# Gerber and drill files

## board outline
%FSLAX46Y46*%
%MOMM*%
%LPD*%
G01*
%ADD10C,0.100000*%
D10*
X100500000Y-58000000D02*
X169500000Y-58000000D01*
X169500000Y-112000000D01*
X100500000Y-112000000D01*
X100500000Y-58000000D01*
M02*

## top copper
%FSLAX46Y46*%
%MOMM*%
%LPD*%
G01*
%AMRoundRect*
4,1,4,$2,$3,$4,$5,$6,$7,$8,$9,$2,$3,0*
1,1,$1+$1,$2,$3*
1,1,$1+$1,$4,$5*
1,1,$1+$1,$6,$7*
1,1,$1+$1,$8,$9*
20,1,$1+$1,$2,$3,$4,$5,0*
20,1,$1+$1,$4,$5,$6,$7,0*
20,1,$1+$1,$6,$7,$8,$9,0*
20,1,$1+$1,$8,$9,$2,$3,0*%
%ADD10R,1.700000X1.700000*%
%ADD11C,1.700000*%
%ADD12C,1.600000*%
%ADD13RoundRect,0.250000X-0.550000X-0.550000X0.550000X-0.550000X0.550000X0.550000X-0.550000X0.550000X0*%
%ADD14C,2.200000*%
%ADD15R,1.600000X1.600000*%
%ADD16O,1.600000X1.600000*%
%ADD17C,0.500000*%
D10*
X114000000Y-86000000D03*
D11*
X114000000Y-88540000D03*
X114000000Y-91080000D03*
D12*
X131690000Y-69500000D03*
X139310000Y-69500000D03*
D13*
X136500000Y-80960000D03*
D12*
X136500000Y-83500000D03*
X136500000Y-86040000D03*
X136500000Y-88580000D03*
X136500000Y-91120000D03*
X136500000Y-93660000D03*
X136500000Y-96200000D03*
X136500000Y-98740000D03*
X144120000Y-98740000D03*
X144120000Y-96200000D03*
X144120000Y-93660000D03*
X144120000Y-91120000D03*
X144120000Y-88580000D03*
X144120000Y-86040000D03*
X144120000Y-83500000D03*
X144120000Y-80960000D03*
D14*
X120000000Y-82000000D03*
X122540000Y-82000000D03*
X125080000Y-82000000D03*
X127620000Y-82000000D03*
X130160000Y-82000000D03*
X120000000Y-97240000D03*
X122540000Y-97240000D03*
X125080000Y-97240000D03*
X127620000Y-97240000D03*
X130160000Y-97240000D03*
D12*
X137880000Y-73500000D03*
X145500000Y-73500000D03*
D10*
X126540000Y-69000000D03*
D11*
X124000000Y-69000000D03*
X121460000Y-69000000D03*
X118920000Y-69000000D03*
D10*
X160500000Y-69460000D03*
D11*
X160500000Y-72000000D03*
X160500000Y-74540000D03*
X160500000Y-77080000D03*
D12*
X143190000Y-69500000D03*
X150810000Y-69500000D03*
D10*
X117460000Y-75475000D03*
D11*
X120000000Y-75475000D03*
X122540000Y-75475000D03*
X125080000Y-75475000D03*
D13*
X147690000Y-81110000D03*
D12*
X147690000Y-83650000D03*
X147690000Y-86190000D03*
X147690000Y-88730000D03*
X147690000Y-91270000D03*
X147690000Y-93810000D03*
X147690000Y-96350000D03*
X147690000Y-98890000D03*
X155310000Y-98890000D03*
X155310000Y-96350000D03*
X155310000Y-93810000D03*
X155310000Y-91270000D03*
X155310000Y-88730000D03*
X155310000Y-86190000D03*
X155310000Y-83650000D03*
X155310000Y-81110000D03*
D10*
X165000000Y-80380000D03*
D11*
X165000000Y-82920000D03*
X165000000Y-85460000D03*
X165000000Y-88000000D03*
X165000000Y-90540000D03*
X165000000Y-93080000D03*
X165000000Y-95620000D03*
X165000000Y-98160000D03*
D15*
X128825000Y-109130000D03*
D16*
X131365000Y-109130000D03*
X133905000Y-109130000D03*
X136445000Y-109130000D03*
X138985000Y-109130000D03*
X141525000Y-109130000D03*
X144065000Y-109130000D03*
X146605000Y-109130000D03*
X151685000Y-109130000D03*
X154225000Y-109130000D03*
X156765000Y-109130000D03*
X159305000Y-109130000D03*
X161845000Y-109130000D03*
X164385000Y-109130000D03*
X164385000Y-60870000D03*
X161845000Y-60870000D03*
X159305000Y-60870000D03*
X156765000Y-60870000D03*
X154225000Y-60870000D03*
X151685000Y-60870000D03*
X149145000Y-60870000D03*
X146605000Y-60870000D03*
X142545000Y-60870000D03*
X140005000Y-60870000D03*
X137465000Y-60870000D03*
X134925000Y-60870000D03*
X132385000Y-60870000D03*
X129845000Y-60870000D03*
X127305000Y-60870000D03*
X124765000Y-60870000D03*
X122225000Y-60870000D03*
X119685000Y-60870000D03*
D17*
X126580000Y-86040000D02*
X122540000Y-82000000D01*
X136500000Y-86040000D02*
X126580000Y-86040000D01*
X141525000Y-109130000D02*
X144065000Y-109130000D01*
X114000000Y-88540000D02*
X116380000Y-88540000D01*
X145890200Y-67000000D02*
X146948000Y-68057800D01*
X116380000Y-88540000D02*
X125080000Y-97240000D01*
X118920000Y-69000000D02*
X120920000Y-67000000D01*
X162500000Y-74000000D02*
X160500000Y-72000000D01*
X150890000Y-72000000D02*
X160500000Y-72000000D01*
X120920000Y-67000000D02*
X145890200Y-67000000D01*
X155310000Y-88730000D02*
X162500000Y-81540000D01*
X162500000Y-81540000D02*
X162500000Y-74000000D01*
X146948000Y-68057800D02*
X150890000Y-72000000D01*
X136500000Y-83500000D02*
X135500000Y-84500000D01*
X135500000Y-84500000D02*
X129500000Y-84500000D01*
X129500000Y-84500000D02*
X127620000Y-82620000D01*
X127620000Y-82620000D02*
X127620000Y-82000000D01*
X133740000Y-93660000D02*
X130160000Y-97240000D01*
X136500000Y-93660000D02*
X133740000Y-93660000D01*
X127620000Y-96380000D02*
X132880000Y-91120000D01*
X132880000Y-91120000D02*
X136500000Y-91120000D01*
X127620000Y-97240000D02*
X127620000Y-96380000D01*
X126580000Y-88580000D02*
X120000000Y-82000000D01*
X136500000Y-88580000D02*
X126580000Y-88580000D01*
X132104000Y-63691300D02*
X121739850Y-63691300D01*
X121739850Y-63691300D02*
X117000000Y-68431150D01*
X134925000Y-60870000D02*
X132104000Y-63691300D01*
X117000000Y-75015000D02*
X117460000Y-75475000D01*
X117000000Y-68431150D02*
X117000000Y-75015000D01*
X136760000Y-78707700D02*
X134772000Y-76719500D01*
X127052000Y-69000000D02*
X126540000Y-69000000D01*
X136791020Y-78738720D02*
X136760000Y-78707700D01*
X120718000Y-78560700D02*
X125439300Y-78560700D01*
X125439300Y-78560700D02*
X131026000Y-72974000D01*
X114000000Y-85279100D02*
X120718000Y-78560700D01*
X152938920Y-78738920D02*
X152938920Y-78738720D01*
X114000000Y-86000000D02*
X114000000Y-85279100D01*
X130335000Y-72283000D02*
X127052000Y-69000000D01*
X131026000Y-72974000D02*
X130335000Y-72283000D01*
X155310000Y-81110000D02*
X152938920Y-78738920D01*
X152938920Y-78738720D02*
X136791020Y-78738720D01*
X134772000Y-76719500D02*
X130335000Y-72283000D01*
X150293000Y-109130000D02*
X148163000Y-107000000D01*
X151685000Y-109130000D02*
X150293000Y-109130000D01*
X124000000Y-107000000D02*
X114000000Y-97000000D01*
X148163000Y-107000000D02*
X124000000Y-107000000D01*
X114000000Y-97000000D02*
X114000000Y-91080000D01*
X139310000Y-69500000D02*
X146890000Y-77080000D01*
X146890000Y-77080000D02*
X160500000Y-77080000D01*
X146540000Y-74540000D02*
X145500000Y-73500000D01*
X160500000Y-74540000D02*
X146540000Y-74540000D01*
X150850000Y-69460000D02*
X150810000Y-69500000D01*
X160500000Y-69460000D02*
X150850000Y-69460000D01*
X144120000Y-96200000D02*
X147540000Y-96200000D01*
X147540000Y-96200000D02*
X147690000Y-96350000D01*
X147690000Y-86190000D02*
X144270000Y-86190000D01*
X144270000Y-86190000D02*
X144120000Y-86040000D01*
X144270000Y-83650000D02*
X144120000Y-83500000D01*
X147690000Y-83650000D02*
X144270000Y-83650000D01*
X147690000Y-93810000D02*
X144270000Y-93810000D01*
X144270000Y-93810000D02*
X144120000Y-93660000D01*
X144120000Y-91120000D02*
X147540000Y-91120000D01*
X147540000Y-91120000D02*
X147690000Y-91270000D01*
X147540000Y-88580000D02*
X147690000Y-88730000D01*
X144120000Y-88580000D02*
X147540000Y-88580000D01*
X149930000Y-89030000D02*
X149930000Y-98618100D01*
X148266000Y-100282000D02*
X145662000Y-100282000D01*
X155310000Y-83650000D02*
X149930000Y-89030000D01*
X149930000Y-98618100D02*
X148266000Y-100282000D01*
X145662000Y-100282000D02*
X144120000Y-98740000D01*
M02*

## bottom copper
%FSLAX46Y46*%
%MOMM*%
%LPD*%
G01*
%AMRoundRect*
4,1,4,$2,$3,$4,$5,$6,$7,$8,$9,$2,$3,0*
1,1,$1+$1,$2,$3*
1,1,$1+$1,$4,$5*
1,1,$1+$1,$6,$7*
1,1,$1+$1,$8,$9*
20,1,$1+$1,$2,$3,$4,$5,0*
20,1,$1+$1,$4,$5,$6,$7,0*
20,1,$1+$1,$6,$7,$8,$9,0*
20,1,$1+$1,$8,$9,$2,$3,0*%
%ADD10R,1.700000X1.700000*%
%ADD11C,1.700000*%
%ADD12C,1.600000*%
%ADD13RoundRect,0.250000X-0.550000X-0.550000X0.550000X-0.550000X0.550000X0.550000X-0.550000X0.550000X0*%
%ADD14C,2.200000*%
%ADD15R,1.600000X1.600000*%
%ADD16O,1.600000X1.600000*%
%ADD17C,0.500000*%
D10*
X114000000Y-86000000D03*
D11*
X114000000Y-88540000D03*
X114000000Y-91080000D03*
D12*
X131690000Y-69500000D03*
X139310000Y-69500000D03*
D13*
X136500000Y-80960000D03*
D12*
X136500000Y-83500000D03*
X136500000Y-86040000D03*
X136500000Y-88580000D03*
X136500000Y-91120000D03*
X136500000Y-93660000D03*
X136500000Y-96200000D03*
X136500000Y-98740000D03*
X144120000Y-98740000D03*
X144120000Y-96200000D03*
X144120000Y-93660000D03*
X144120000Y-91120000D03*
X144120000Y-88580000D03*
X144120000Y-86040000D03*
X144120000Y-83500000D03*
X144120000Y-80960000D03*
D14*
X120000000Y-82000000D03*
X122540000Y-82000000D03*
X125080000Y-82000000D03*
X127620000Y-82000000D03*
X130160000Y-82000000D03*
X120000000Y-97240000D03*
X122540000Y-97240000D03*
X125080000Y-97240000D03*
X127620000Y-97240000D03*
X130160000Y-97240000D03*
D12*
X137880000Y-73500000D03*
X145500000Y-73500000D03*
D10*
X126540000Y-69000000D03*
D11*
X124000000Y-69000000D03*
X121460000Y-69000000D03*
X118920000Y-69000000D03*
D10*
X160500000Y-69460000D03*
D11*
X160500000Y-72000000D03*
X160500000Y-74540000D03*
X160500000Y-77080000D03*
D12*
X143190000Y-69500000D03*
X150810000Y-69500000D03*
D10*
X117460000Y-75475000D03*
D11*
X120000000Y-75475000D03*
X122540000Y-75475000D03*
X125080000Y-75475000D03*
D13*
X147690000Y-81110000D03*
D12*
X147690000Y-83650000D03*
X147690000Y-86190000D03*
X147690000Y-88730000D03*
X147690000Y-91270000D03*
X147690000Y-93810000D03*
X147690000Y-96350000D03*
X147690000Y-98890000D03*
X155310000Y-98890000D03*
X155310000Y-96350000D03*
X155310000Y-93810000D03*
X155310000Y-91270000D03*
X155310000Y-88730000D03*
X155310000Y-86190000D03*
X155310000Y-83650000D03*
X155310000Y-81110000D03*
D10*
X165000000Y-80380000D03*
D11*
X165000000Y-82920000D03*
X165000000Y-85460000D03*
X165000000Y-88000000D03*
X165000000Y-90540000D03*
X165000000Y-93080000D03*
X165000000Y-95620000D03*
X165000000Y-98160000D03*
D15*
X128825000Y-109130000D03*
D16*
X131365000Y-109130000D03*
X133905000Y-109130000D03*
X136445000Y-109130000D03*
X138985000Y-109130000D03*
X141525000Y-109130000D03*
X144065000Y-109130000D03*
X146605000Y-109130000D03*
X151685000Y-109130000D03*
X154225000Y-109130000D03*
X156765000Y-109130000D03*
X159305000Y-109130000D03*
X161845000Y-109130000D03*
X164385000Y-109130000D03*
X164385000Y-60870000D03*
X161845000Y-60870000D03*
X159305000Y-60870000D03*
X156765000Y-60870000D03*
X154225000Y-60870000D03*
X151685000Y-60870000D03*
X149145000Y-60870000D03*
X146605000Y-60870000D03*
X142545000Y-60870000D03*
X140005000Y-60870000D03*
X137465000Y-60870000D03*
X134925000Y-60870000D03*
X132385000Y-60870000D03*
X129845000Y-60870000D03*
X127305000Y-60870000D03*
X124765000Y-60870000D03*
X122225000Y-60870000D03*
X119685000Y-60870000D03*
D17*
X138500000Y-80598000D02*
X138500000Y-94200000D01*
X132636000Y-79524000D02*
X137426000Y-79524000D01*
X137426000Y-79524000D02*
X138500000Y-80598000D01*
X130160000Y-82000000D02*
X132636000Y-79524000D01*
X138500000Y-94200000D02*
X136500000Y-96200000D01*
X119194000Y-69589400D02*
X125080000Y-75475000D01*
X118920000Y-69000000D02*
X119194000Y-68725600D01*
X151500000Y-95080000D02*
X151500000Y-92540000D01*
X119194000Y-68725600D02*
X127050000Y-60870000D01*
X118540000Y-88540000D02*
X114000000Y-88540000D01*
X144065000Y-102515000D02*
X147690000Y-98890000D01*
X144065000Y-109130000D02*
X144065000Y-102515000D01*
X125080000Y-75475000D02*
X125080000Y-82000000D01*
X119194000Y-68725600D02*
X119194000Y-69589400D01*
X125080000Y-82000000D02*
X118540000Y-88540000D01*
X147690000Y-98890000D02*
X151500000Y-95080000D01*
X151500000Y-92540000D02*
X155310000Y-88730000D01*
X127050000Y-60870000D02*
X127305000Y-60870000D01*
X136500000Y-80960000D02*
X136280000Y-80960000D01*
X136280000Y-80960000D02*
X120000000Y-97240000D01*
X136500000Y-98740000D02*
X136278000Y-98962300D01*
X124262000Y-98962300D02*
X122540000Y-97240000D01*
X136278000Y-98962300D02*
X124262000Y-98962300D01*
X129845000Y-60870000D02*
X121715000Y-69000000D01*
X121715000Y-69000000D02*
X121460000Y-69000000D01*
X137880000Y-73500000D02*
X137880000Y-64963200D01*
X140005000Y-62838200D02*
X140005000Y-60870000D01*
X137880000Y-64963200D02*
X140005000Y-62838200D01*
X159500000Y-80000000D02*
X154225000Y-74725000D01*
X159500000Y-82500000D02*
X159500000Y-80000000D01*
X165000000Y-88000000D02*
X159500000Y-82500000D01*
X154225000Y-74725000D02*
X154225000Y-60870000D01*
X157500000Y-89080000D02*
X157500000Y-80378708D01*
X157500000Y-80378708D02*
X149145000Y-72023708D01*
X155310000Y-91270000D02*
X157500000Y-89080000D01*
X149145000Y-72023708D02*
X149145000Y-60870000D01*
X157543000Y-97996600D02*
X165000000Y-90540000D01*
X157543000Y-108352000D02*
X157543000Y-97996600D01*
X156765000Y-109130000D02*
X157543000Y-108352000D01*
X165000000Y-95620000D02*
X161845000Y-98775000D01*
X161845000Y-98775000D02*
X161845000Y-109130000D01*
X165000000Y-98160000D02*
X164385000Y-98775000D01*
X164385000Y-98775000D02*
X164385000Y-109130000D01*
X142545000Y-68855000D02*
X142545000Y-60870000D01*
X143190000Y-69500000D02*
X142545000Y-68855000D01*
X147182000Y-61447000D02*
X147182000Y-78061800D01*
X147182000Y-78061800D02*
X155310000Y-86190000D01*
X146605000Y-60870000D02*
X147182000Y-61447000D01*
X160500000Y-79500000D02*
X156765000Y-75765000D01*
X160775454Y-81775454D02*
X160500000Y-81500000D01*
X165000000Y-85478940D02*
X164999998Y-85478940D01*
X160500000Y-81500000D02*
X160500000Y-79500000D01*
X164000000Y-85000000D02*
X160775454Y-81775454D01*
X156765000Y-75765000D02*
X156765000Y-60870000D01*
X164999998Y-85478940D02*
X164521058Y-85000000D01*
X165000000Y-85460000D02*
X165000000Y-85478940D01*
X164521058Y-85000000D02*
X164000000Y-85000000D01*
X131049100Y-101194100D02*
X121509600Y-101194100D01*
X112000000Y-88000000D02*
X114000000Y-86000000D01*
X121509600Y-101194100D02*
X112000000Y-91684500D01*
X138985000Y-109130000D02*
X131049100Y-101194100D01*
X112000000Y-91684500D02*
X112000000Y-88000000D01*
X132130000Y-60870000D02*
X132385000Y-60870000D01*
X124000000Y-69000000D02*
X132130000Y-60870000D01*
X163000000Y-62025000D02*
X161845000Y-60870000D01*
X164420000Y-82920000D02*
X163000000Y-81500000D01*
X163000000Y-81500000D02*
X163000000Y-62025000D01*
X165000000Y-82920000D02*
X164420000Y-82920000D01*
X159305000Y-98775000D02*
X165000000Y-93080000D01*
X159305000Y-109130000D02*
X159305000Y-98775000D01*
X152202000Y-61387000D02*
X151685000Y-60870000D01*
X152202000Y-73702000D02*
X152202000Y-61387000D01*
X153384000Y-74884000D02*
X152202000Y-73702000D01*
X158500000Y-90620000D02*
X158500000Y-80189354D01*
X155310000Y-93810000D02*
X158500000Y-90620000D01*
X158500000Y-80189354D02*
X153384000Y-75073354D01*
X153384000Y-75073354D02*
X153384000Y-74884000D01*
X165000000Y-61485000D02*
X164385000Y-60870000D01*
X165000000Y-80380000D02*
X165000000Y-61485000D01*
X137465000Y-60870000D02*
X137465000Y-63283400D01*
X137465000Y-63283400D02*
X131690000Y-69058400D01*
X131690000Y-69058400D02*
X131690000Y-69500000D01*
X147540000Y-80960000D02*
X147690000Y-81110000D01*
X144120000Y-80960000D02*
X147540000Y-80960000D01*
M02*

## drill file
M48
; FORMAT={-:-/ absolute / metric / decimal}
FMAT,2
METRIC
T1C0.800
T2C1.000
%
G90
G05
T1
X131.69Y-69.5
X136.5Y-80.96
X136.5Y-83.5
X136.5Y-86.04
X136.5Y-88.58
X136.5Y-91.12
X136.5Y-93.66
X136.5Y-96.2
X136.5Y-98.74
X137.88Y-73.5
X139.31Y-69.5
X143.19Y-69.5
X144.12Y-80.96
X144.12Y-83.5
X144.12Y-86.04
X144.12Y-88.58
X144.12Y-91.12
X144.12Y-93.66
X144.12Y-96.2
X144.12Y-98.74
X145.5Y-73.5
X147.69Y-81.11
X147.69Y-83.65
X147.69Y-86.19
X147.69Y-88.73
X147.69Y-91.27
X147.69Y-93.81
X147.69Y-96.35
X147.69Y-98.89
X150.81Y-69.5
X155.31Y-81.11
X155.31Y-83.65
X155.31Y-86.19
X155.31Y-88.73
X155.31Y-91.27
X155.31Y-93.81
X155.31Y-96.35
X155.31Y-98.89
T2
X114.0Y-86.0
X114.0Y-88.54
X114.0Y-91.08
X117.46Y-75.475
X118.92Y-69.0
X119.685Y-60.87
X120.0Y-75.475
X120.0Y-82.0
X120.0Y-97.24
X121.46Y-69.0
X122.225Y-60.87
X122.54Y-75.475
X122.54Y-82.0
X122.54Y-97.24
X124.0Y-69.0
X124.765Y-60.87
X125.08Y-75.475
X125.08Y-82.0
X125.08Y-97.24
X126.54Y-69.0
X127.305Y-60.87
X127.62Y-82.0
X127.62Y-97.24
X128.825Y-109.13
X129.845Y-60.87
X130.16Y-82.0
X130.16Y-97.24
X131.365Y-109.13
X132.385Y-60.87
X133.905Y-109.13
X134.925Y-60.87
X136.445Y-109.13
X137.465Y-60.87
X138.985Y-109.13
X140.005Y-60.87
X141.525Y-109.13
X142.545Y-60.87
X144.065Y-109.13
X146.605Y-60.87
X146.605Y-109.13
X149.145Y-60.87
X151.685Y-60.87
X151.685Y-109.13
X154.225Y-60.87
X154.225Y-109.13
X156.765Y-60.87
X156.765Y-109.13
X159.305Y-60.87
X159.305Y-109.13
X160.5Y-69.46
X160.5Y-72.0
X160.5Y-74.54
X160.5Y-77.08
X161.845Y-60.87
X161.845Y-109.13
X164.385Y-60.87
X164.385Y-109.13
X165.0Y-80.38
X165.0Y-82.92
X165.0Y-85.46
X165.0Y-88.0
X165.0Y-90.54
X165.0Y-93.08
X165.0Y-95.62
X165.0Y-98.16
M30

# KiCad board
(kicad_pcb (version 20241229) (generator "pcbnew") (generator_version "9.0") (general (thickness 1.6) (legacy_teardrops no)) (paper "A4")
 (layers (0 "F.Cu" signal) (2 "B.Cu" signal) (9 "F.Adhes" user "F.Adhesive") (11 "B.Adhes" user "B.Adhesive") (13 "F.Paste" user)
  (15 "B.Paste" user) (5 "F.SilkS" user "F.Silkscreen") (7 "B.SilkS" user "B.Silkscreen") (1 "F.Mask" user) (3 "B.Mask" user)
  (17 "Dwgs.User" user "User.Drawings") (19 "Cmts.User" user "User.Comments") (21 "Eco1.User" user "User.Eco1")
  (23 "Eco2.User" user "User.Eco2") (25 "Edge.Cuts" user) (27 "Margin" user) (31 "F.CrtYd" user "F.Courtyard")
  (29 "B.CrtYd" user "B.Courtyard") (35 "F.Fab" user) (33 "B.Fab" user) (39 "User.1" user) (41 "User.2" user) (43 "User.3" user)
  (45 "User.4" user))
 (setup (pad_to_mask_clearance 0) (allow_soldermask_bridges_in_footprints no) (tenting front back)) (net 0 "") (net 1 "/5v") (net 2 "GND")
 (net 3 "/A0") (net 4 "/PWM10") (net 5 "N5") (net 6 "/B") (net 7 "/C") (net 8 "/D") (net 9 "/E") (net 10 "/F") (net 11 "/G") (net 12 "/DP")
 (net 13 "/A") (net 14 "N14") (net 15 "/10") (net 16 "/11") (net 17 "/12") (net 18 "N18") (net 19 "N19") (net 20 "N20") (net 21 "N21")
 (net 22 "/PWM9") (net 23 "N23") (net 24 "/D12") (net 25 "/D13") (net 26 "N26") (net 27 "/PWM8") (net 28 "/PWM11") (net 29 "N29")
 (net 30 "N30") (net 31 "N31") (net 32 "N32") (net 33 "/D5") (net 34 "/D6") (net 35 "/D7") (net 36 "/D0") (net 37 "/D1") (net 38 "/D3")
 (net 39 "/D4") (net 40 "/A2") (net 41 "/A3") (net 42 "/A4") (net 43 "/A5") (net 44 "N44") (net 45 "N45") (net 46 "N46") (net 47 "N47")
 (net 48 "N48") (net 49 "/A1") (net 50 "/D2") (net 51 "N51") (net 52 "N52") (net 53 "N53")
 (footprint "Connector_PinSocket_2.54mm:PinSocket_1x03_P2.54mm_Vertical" (layer "F.Cu") (at 114 86)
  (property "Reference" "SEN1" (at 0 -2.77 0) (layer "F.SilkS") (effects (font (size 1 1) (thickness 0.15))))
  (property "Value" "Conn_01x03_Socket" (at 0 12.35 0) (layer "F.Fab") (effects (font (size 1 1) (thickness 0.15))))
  (pad "1" thru_hole rect (at 0 0) (size 1.7 1.7) (drill 1) (layers "*.Cu" "*.Mask") (remove_unused_layers no) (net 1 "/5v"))
  (pad "2" thru_hole circle (at 0 2.54) (size 1.7 1.7) (drill 1) (layers "*.Cu" "*.Mask") (remove_unused_layers no) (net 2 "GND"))
  (pad "3" thru_hole circle (at 0 5.08) (size 1.7 1.7) (drill 1) (layers "*.Cu" "*.Mask") (remove_unused_layers no) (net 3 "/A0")))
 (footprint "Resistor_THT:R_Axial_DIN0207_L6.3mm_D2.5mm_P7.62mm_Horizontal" (layer "F.Cu") (at 131.69 69.5)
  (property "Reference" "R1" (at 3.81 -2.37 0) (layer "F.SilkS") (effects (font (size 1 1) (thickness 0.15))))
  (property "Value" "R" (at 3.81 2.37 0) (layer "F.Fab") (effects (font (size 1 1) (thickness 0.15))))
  (pad "1" thru_hole circle (at 0 0) (size 1.6 1.6) (drill 0.8) (layers "*.Cu" "*.Mask") (remove_unused_layers no) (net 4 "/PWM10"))
  (pad "2" thru_hole circle (at 7.62 0) (size 1.6 1.6) (drill 0.8) (layers "*.Cu" "*.Mask") (remove_unused_layers no) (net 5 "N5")))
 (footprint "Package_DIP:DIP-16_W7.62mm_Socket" (layer "F.Cu") (at 136.5 80.96)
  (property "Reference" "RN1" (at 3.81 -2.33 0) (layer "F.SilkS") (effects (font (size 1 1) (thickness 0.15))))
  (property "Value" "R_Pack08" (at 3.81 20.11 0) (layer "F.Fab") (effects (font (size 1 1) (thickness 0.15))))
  (pad "1" thru_hole roundrect (at 0 0) (size 1.6 1.6) (drill 0.8) (layers "*.Cu" "*.Mask") (remove_unused_layers no)
   (roundrect_rratio 0.15625) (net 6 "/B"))
  (pad "2" thru_hole circle (at 0 2.54) (size 1.6 1.6) (drill 0.8) (layers "*.Cu" "*.Mask") (remove_unused_layers no) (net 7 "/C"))
  (pad "3" thru_hole circle (at 0 5.08) (size 1.6 1.6) (drill 0.8) (layers "*.Cu" "*.Mask") (remove_unused_layers no) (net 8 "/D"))
  (pad "4" thru_hole circle (at 0 7.62) (size 1.6 1.6) (drill 0.8) (layers "*.Cu" "*.Mask") (remove_unused_layers no) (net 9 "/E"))
  (pad "5" thru_hole circle (at 0 10.16) (size 1.6 1.6) (drill 0.8) (layers "*.Cu" "*.Mask") (remove_unused_layers no) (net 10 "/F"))
  (pad "6" thru_hole circle (at 0 12.7) (size 1.6 1.6) (drill 0.8) (layers "*.Cu" "*.Mask") (remove_unused_layers no) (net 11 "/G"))
  (pad "7" thru_hole circle (at 0 15.24) (size 1.6 1.6) (drill 0.8) (layers "*.Cu" "*.Mask") (remove_unused_layers no) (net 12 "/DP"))
  (pad "8" thru_hole circle (at 0 17.78) (size 1.6 1.6) (drill 0.8) (layers "*.Cu" "*.Mask") (remove_unused_layers no) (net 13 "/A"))
  (pad "9" thru_hole circle (at 7.62 17.78) (size 1.6 1.6) (drill 0.8) (layers "*.Cu" "*.Mask") (remove_unused_layers no) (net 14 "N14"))
  (pad "10" thru_hole circle (at 7.62 15.24) (size 1.6 1.6) (drill 0.8) (layers "*.Cu" "*.Mask") (remove_unused_layers no) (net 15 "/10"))
  (pad "11" thru_hole circle (at 7.62 12.7) (size 1.6 1.6) (drill 0.8) (layers "*.Cu" "*.Mask") (remove_unused_layers no) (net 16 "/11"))
  (pad "12" thru_hole circle (at 7.62 10.16) (size 1.6 1.6) (drill 0.8) (layers "*.Cu" "*.Mask") (remove_unused_layers no) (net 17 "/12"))
  (pad "13" thru_hole circle (at 7.62 7.62) (size 1.6 1.6) (drill 0.8) (layers "*.Cu" "*.Mask") (remove_unused_layers no) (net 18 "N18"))
  (pad "14" thru_hole circle (at 7.62 5.08) (size 1.6 1.6) (drill 0.8) (layers "*.Cu" "*.Mask") (remove_unused_layers no) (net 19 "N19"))
  (pad "15" thru_hole circle (at 7.62 2.54) (size 1.6 1.6) (drill 0.8) (layers "*.Cu" "*.Mask") (remove_unused_layers no) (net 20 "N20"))
  (pad "16" thru_hole circle (at 7.62 0) (size 1.6 1.6) (drill 0.8) (layers "*.Cu" "*.Mask") (remove_unused_layers no) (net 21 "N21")))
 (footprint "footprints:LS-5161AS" (layer "F.Cu") (at 120 82)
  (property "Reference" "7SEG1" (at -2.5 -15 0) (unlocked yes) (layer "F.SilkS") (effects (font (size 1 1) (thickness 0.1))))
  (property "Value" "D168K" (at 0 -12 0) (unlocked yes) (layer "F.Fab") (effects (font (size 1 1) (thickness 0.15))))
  (pad "1" thru_hole circle (at 0 0) (size 2.2 2.2) (drill 1) (layers "*.Cu" "*.Mask") (remove_unused_layers no) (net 9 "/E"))
  (pad "2" thru_hole circle (at 2.54 0) (size 2.2 2.2) (drill 1) (layers "*.Cu" "*.Mask") (remove_unused_layers no) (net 8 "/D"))
  (pad "3" thru_hole circle (at 5.08 0) (size 2.2 2.2) (drill 1) (layers "*.Cu" "*.Mask") (remove_unused_layers no) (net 2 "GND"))
  (pad "4" thru_hole circle (at 7.62 0) (size 2.2 2.2) (drill 1) (layers "*.Cu" "*.Mask") (remove_unused_layers no) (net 7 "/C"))
  (pad "5" thru_hole circle (at 10.16 0) (size 2.2 2.2) (drill 1) (layers "*.Cu" "*.Mask") (remove_unused_layers no) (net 12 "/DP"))
  (pad "6" thru_hole circle (at 0 15.24) (size 2.2 2.2) (drill 1) (layers "*.Cu" "*.Mask") (remove_unused_layers no) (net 6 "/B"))
  (pad "7" thru_hole circle (at 2.54 15.24) (size 2.2 2.2) (drill 1) (layers "*.Cu" "*.Mask") (remove_unused_layers no) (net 13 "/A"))
  (pad "8" thru_hole circle (at 5.08 15.24) (size 2.2 2.2) (drill 1) (layers "*.Cu" "*.Mask") (remove_unused_layers no) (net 2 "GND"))
  (pad "9" thru_hole circle (at 7.62 15.24) (size 2.2 2.2) (drill 1) (layers "*.Cu" "*.Mask") (remove_unused_layers no) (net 10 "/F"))
  (pad "10" thru_hole circle (at 10.16 15.24) (size 2.2 2.2) (drill 1) (layers "*.Cu" "*.Mask") (remove_unused_layers no) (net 11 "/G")))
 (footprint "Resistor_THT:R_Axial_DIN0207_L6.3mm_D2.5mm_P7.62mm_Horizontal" (layer "F.Cu") (at 137.88 73.5)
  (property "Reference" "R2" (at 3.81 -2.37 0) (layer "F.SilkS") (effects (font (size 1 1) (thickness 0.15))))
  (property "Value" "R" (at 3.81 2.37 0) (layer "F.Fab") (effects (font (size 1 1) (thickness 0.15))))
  (pad "1" thru_hole circle (at 0 0) (size 1.6 1.6) (drill 0.8) (layers "*.Cu" "*.Mask") (remove_unused_layers no) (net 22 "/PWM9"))
  (pad "2" thru_hole circle (at 7.62 0) (size 1.6 1.6) (drill 0.8) (layers "*.Cu" "*.Mask") (remove_unused_layers no) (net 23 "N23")))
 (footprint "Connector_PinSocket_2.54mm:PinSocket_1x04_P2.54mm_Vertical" (layer "F.Cu") (at 126.54 69 -90)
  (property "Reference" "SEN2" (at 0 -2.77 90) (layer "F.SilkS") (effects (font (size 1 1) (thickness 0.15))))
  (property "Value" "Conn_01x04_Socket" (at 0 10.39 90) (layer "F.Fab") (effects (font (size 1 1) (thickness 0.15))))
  (pad "1" thru_hole rect (at 0 0 270) (size 1.7 1.7) (drill 1) (layers "*.Cu" "*.Mask") (remove_unused_layers no) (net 1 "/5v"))
  (pad "2" thru_hole circle (at 0 2.54 270) (size 1.7 1.7) (drill 1) (layers "*.Cu" "*.Mask") (remove_unused_layers no) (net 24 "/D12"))
  (pad "3" thru_hole circle (at 0 5.08 270) (size 1.7 1.7) (drill 1) (layers "*.Cu" "*.Mask") (remove_unused_layers no) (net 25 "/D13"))
  (pad "4" thru_hole circle (at 0 7.62 270) (size 1.7 1.7) (drill 1) (layers "*.Cu" "*.Mask") (remove_unused_layers no) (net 2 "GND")))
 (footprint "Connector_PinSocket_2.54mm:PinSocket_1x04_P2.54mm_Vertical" (layer "F.Cu") (at 160.5 69.46)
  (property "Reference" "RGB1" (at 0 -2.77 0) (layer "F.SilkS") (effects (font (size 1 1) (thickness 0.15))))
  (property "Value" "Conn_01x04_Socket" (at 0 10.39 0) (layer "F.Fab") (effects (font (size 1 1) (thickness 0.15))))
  (pad "1" thru_hole rect (at 0 0) (size 1.7 1.7) (drill 1) (layers "*.Cu" "*.Mask") (remove_unused_layers no) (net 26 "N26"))
  (pad "2" thru_hole circle (at 0 2.54) (size 1.7 1.7) (drill 1) (layers "*.Cu" "*.Mask") (remove_unused_layers no) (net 2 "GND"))
  (pad "3" thru_hole circle (at 0 5.08) (size 1.7 1.7) (drill 1) (layers "*.Cu" "*.Mask") (remove_unused_layers no) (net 23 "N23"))
  (pad "4" thru_hole circle (at 0 7.62) (size 1.7 1.7) (drill 1) (layers "*.Cu" "*.Mask") (remove_unused_layers no) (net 5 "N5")))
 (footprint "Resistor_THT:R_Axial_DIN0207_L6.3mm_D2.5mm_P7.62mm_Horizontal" (layer "F.Cu") (at 143.19 69.5)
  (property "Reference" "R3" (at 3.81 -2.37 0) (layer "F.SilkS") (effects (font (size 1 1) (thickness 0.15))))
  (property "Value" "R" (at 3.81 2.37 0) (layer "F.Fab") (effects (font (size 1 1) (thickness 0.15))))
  (pad "1" thru_hole circle (at 0 0) (size 1.6 1.6) (drill 0.8) (layers "*.Cu" "*.Mask") (remove_unused_layers no) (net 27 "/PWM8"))
  (pad "2" thru_hole circle (at 7.62 0) (size 1.6 1.6) (drill 0.8) (layers "*.Cu" "*.Mask") (remove_unused_layers no) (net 26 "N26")))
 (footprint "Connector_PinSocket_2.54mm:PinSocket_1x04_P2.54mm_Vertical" (layer "F.Cu") (at 117.46 75.475 90)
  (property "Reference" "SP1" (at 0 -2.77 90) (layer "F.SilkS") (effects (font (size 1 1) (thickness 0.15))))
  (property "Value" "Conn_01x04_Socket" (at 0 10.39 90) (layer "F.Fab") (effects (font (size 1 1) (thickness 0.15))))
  (pad "1" thru_hole rect (at 0 0 90) (size 1.7 1.7) (drill 1) (layers "*.Cu" "*.Mask") (remove_unused_layers no) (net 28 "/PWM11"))
  (pad "2" thru_hole circle (at 0 2.54 90) (size 1.7 1.7) (drill 1) (layers "*.Cu" "*.Mask") (remove_unused_layers no) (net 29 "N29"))
  (pad "3" thru_hole circle (at 0 5.08 90) (size 1.7 1.7) (drill 1) (layers "*.Cu" "*.Mask") (remove_unused_layers no) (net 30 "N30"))
  (pad "4" thru_hole circle (at 0 7.62 90) (size 1.7 1.7) (drill 1) (layers "*.Cu" "*.Mask") (remove_unused_layers no) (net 2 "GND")))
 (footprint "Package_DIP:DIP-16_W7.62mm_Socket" (layer "F.Cu") (at 147.69 81.11)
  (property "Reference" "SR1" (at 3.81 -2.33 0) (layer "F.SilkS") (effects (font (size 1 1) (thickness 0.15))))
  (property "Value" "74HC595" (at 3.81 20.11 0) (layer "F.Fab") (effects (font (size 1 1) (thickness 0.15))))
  (pad "1" thru_hole roundrect (at 0 0) (size 1.6 1.6) (drill 0.8) (layers "*.Cu" "*.Mask") (remove_unused_layers no)
   (roundrect_rratio 0.15625) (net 21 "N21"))
  (pad "2" thru_hole circle (at 0 2.54) (size 1.6 1.6) (drill 0.8) (layers "*.Cu" "*.Mask") (remove_unused_layers no) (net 20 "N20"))
  (pad "3" thru_hole circle (at 0 5.08) (size 1.6 1.6) (drill 0.8) (layers "*.Cu" "*.Mask") (remove_unused_layers no) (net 19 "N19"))
  (pad "4" thru_hole circle (at 0 7.62) (size 1.6 1.6) (drill 0.8) (layers "*.Cu" "*.Mask") (remove_unused_layers no) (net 18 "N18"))
  (pad "5" thru_hole circle (at 0 10.16) (size 1.6 1.6) (drill 0.8) (layers "*.Cu" "*.Mask") (remove_unused_layers no) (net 17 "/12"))
  (pad "6" thru_hole circle (at 0 12.7) (size 1.6 1.6) (drill 0.8) (layers "*.Cu" "*.Mask") (remove_unused_layers no) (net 16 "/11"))
  (pad "7" thru_hole circle (at 0 15.24) (size 1.6 1.6) (drill 0.8) (layers "*.Cu" "*.Mask") (remove_unused_layers no) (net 15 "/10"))
  (pad "8" thru_hole circle (at 0 17.78) (size 1.6 1.6) (drill 0.8) (layers "*.Cu" "*.Mask") (remove_unused_layers no) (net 2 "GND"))
  (pad "9" thru_hole circle (at 7.62 17.78) (size 1.6 1.6) (drill 0.8) (layers "*.Cu" "*.Mask") (remove_unused_layers no) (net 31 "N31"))
  (pad "10" thru_hole circle (at 7.62 15.24) (size 1.6 1.6) (drill 0.8) (layers "*.Cu" "*.Mask") (remove_unused_layers no) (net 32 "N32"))
  (pad "11" thru_hole circle (at 7.62 12.7) (size 1.6 1.6) (drill 0.8) (layers "*.Cu" "*.Mask") (remove_unused_layers no) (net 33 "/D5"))
  (pad "12" thru_hole circle (at 7.62 10.16) (size 1.6 1.6) (drill 0.8) (layers "*.Cu" "*.Mask") (remove_unused_layers no) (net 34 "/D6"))
  (pad "13" thru_hole circle (at 7.62 7.62) (size 1.6 1.6) (drill 0.8) (layers "*.Cu" "*.Mask") (remove_unused_layers no) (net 2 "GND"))
  (pad "14" thru_hole circle (at 7.62 5.08) (size 1.6 1.6) (drill 0.8) (layers "*.Cu" "*.Mask") (remove_unused_layers no) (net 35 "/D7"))
  (pad "15" thru_hole circle (at 7.62 2.54) (size 1.6 1.6) (drill 0.8) (layers "*.Cu" "*.Mask") (remove_unused_layers no) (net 14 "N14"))
  (pad "16" thru_hole circle (at 7.62 0) (size 1.6 1.6) (drill 0.8) (layers "*.Cu" "*.Mask") (remove_unused_layers no) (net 1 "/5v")))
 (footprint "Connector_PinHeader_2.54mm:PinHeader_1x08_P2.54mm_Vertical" (layer "F.Cu") (at 165 80.38)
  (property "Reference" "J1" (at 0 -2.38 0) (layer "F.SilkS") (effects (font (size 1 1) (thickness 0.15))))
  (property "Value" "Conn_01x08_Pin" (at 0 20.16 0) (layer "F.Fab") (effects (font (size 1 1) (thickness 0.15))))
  (pad "1" thru_hole rect (at 0 0) (size 1.7 1.7) (drill 1) (layers "*.Cu" "*.Mask") (remove_unused_layers no) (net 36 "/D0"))
  (pad "2" thru_hole circle (at 0 2.54) (size 1.7 1.7) (drill 1) (layers "*.Cu" "*.Mask") (remove_unused_layers no) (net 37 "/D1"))
  (pad "3" thru_hole circle (at 0 5.08) (size 1.7 1.7) (drill 1) (layers "*.Cu" "*.Mask") (remove_unused_layers no) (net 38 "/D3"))
  (pad "4" thru_hole circle (at 0 7.62) (size 1.7 1.7) (drill 1) (layers "*.Cu" "*.Mask") (remove_unused_layers no) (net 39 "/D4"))
  (pad "5" thru_hole circle (at 0 10.16) (size 1.7 1.7) (drill 1) (layers "*.Cu" "*.Mask") (remove_unused_layers no) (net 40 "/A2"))
  (pad "6" thru_hole circle (at 0 12.7) (size 1.7 1.7) (drill 1) (layers "*.Cu" "*.Mask") (remove_unused_layers no) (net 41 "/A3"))
  (pad "7" thru_hole circle (at 0 15.24) (size 1.7 1.7) (drill 1) (layers "*.Cu" "*.Mask") (remove_unused_layers no) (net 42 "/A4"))
  (pad "8" thru_hole circle (at 0 17.78) (size 1.7 1.7) (drill 1) (layers "*.Cu" "*.Mask") (remove_unused_layers no) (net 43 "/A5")))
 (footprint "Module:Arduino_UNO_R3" (layer "B.Cu") (at 128.825 109.13)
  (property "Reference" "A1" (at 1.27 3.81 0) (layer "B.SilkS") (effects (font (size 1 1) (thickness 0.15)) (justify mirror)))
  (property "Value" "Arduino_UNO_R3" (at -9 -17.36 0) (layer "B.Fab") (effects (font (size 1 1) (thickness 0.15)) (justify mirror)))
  (pad "1" thru_hole rect (at 0 0 270) (size 1.6 1.6) (drill 1) (layers "*.Cu" "*.Mask") (remove_unused_layers no) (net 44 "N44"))
  (pad "2" thru_hole oval (at 2.54 0 270) (size 1.6 1.6) (drill 1) (layers "*.Cu" "*.Mask") (remove_unused_layers no) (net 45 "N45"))
  (pad "3" thru_hole oval (at 5.08 0 270) (size 1.6 1.6) (drill 1) (layers "*.Cu" "*.Mask") (remove_unused_layers no) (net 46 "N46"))
  (pad "4" thru_hole oval (at 7.62 0 270) (size 1.6 1.6) (drill 1) (layers "*.Cu" "*.Mask") (remove_unused_layers no) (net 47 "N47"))
  (pad "5" thru_hole oval (at 10.16 0 270) (size 1.6 1.6) (drill 1) (layers "*.Cu" "*.Mask") (remove_unused_layers no) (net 1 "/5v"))
  (pad "6" thru_hole oval (at 12.7 0 270) (size 1.6 1.6) (drill 1) (layers "*.Cu" "*.Mask") (remove_unused_layers no) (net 2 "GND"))
  (pad "7" thru_hole oval (at 15.24 0 270) (size 1.6 1.6) (drill 1) (layers "*.Cu" "*.Mask") (remove_unused_layers no) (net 2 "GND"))
  (pad "8" thru_hole oval (at 17.78 0 270) (size 1.6 1.6) (drill 1) (layers "*.Cu" "*.Mask") (remove_unused_layers no) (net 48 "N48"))
  (pad "9" thru_hole oval (at 22.86 0 270) (size 1.6 1.6) (drill 1) (layers "*.Cu" "*.Mask") (remove_unused_layers no) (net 3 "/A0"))
  (pad "10" thru_hole oval (at 25.4 0 270) (size 1.6 1.6) (drill 1) (layers "*.Cu" "*.Mask") (remove_unused_layers no) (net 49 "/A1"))
  (pad "11" thru_hole oval (at 27.94 0 270) (size 1.6 1.6) (drill 1) (layers "*.Cu" "*.Mask") (remove_unused_layers no) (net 40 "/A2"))
  (pad "12" thru_hole oval (at 30.48 0 270) (size 1.6 1.6) (drill 1) (layers "*.Cu" "*.Mask") (remove_unused_layers no) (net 41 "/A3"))
  (pad "13" thru_hole oval (at 33.02 0 270) (size 1.6 1.6) (drill 1) (layers "*.Cu" "*.Mask") (remove_unused_layers no) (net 42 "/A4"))
  (pad "14" thru_hole oval (at 35.56 0 270) (size 1.6 1.6) (drill 1) (layers "*.Cu" "*.Mask") (remove_unused_layers no) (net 43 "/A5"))
  (pad "15" thru_hole oval (at 35.56 -48.26 270) (size 1.6 1.6) (drill 1) (layers "*.Cu" "*.Mask") (remove_unused_layers no) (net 36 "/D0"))
  (pad "16" thru_hole oval (at 33.02 -48.26 270) (size 1.6 1.6) (drill 1) (layers "*.Cu" "*.Mask") (remove_unused_layers no) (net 37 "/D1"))
  (pad "17" thru_hole oval (at 30.48 -48.26 270) (size 1.6 1.6) (drill 1) (layers "*.Cu" "*.Mask") (remove_unused_layers no) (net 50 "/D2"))
  (pad "18" thru_hole oval (at 27.94 -48.26 270) (size 1.6 1.6) (drill 1) (layers "*.Cu" "*.Mask") (remove_unused_layers no) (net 38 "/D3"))
  (pad "19" thru_hole oval (at 25.4 -48.26 270) (size 1.6 1.6) (drill 1) (layers "*.Cu" "*.Mask") (remove_unused_layers no) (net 39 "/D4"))
  (pad "20" thru_hole oval (at 22.86 -48.26 270) (size 1.6 1.6) (drill 1) (layers "*.Cu" "*.Mask") (remove_unused_layers no) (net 33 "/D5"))
  (pad "21" thru_hole oval (at 20.32 -48.26 270) (size 1.6 1.6) (drill 1) (layers "*.Cu" "*.Mask") (remove_unused_layers no) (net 34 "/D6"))
  (pad "22" thru_hole oval (at 17.78 -48.26 270) (size 1.6 1.6) (drill 1) (layers "*.Cu" "*.Mask") (remove_unused_layers no) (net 35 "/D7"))
  (pad "23" thru_hole oval (at 13.72 -48.26 270) (size 1.6 1.6) (drill 1) (layers "*.Cu" "*.Mask") (remove_unused_layers no)
   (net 27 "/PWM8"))
  (pad "24" thru_hole oval (at 11.18 -48.26 270) (size 1.6 1.6) (drill 1) (layers "*.Cu" "*.Mask") (remove_unused_layers no)
   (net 22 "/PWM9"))
  (pad "25" thru_hole oval (at 8.64 -48.26 270) (size 1.6 1.6) (drill 1) (layers "*.Cu" "*.Mask") (remove_unused_layers no) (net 4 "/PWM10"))
  (pad "26" thru_hole oval (at 6.1 -48.26 270) (size 1.6 1.6) (drill 1) (layers "*.Cu" "*.Mask") (remove_unused_layers no) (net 28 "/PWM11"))
  (pad "27" thru_hole oval (at 3.56 -48.26 270) (size 1.6 1.6) (drill 1) (layers "*.Cu" "*.Mask") (remove_unused_layers no) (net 24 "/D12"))
  (pad "28" thru_hole oval (at 1.02 -48.26 270) (size 1.6 1.6) (drill 1) (layers "*.Cu" "*.Mask") (remove_unused_layers no) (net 25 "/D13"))
  (pad "29" thru_hole oval (at -1.52 -48.26 270) (size 1.6 1.6) (drill 1) (layers "*.Cu" "*.Mask") (remove_unused_layers no) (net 2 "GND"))
  (pad "30" thru_hole oval (at -4.06 -48.26 270) (size 1.6 1.6) (drill 1) (layers "*.Cu" "*.Mask") (remove_unused_layers no) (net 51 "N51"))
  (pad "31" thru_hole oval (at -6.6 -48.26 270) (size 1.6 1.6) (drill 1) (layers "*.Cu" "*.Mask") (remove_unused_layers no) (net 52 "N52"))
  (pad "32" thru_hole oval (at -9.14 -48.26 270) (size 1.6 1.6) (drill 1) (layers "*.Cu" "*.Mask") (remove_unused_layers no) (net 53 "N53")))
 (gr_rect (start 100.5 58) (end 169.5 112) (stroke (width 0.1) (type default)) (fill no) (layer "Edge.Cuts"))
 (segment (start 138.5 80.598) (end 138.5 94.2) (width 0.5) (layer "B.Cu") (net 12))
 (segment (start 132.636 79.524) (end 137.426 79.524) (width 0.5) (layer "B.Cu") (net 12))
 (segment (start 137.426 79.524) (end 138.5 80.598) (width 0.5) (layer "B.Cu") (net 12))
 (segment (start 130.16 82) (end 132.636 79.524) (width 0.5) (layer "B.Cu") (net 12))
 (segment (start 138.5 94.2) (end 136.5 96.2) (width 0.5) (layer "B.Cu") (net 12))
 (segment (start 126.58 86.04) (end 122.54 82) (width 0.5) (layer "F.Cu") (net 8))
 (segment (start 136.5 86.04) (end 126.58 86.04) (width 0.5) (layer "F.Cu") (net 8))
 (segment (start 141.525 109.13) (end 144.065 109.13) (width 0.5) (layer "F.Cu") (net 2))
 (segment (start 114 88.54) (end 116.38 88.54) (width 0.5) (layer "F.Cu") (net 2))
 (segment (start 145.8902 67) (end 146.948 68.0578) (width 0.5) (layer "F.Cu") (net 2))
 (segment (start 116.38 88.54) (end 125.08 97.24) (width 0.5) (layer "F.Cu") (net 2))
 (segment (start 118.92 69) (end 120.92 67) (width 0.5) (layer "F.Cu") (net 2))
 (segment (start 162.5 74) (end 160.5 72) (width 0.5) (layer "F.Cu") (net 2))
 (segment (start 150.89 72) (end 160.5 72) (width 0.5) (layer "F.Cu") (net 2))
 (segment (start 120.92 67) (end 145.8902 67) (width 0.5) (layer "F.Cu") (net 2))
 (segment (start 155.31 88.73) (end 162.5 81.54) (width 0.5) (layer "F.Cu") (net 2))
 (segment (start 162.5 81.54) (end 162.5 74) (width 0.5) (layer "F.Cu") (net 2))
 (segment (start 146.948 68.0578) (end 150.89 72) (width 0.5) (layer "F.Cu") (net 2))
 (segment (start 119.194 69.5894) (end 125.08 75.475) (width 0.5) (layer "B.Cu") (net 2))
 (segment (start 118.92 69) (end 119.194 68.7256) (width 0.5) (layer "B.Cu") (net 2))
 (segment (start 151.5 95.08) (end 151.5 92.54) (width 0.5) (layer "B.Cu") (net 2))
 (segment (start 119.194 68.7256) (end 127.05 60.87) (width 0.5) (layer "B.Cu") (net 2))
 (segment (start 118.54 88.54) (end 114 88.54) (width 0.5) (layer "B.Cu") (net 2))
 (segment (start 144.065 102.515) (end 147.69 98.89) (width 0.5) (layer "B.Cu") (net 2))
 (segment (start 144.065 109.13) (end 144.065 102.515) (width 0.5) (layer "B.Cu") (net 2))
 (segment (start 125.08 75.475) (end 125.08 82) (width 0.5) (layer "B.Cu") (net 2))
 (segment (start 119.194 68.7256) (end 119.194 69.5894) (width 0.5) (layer "B.Cu") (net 2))
 (segment (start 125.08 82) (end 118.54 88.54) (width 0.5) (layer "B.Cu") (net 2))
 (segment (start 147.69 98.89) (end 151.5 95.08) (width 0.5) (layer "B.Cu") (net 2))
 (segment (start 151.5 92.54) (end 155.31 88.73) (width 0.5) (layer "B.Cu") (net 2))
 (segment (start 127.05 60.87) (end 127.305 60.87) (width 0.5) (layer "B.Cu") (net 2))
 (segment (start 136.5 83.5) (end 135.5 84.5) (width 0.5) (layer "F.Cu") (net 7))
 (segment (start 135.5 84.5) (end 129.5 84.5) (width 0.5) (layer "F.Cu") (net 7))
 (segment (start 129.5 84.5) (end 127.62 82.62) (width 0.5) (layer "F.Cu") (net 7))
 (segment (start 127.62 82.62) (end 127.62 82) (width 0.5) (layer "F.Cu") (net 7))
 (segment (start 136.5 80.96) (end 136.28 80.96) (width 0.5) (layer "B.Cu") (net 6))
 (segment (start 136.28 80.96) (end 120 97.24) (width 0.5) (layer "B.Cu") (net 6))
 (segment (start 136.5 98.74) (end 136.278 98.9623) (width 0.5) (layer "B.Cu") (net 13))
 (segment (start 124.262 98.9623) (end 122.54 97.24) (width 0.5) (layer "B.Cu") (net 13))
 (segment (start 136.278 98.9623) (end 124.262 98.9623) (width 0.5) (layer "B.Cu") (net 13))
 (segment (start 133.74 93.66) (end 130.16 97.24) (width 0.5) (layer "F.Cu") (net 11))
 (segment (start 136.5 93.66) (end 133.74 93.66) (width 0.5) (layer "F.Cu") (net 11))
 (segment (start 127.62 96.38) (end 132.88 91.12) (width 0.5) (layer "F.Cu") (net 10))
 (segment (start 132.88 91.12) (end 136.5 91.12) (width 0.5) (layer "F.Cu") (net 10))
 (segment (start 127.62 97.24) (end 127.62 96.38) (width 0.5) (layer "F.Cu") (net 10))
 (segment (start 126.58 88.58) (end 120 82) (width 0.5) (layer "F.Cu") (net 9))
 (segment (start 136.5 88.58) (end 126.58 88.58) (width 0.5) (layer "F.Cu") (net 9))
 (segment (start 129.845 60.87) (end 121.715 69) (width 0.5) (layer "B.Cu") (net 25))
 (segment (start 121.715 69) (end 121.46 69) (width 0.5) (layer "B.Cu") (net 25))
 (segment (start 137.88 73.5) (end 137.88 64.9632) (width 0.5) (layer "B.Cu") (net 22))
 (segment (start 140.005 62.8382) (end 140.005 60.87) (width 0.5) (layer "B.Cu") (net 22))
 (segment (start 137.88 64.9632) (end 140.005 62.8382) (width 0.5) (layer "B.Cu") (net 22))
 (segment (start 159.5 80) (end 154.225 74.725) (width 0.5) (layer "B.Cu") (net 39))
 (segment (start 159.5 82.5) (end 159.5 80) (width 0.5) (layer "B.Cu") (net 39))
 (segment (start 165 88) (end 159.5 82.5) (width 0.5) (layer "B.Cu") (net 39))
 (segment (start 154.225 74.725) (end 154.225 60.87) (width 0.5) (layer "B.Cu") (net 39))
 (segment (start 157.5 89.08) (end 157.5 80.378708) (width 0.5) (layer "B.Cu") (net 34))
 (segment (start 157.5 80.378708) (end 149.145 72.023708) (width 0.5) (layer "B.Cu") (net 34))
 (segment (start 155.31 91.27) (end 157.5 89.08) (width 0.5) (layer "B.Cu") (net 34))
 (segment (start 149.145 72.023708) (end 149.145 60.87) (width 0.5) (layer "B.Cu") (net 34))
 (segment (start 157.543 97.9966) (end 165 90.54) (width 0.5) (layer "B.Cu") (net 40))
 (segment (start 157.543 108.352) (end 157.543 97.9966) (width 0.5) (layer "B.Cu") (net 40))
 (segment (start 156.765 109.13) (end 157.543 108.352) (width 0.5) (layer "B.Cu") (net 40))
 (segment (start 165 95.62) (end 161.845 98.775) (width 0.5) (layer "B.Cu") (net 42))
 (segment (start 161.845 98.775) (end 161.845 109.13) (width 0.5) (layer "B.Cu") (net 42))
 (segment (start 165 98.16) (end 164.385 98.775) (width 0.5) (layer "B.Cu") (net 43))
 (segment (start 164.385 98.775) (end 164.385 109.13) (width 0.5) (layer "B.Cu") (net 43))
 (segment (start 132.104 63.6913) (end 121.73985 63.6913) (width 0.5) (layer "F.Cu") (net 28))
 (segment (start 121.73985 63.6913) (end 117 68.43115) (width 0.5) (layer "F.Cu") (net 28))
 (segment (start 134.925 60.87) (end 132.104 63.6913) (width 0.5) (layer "F.Cu") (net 28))
 (segment (start 117 75.015) (end 117.46 75.475) (width 0.5) (layer "F.Cu") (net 28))
 (segment (start 117 68.43115) (end 117 75.015) (width 0.5) (layer "F.Cu") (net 28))
 (segment (start 142.545 68.855) (end 142.545 60.87) (width 0.5) (layer "B.Cu") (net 27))
 (segment (start 143.19 69.5) (end 142.545 68.855) (width 0.5) (layer "B.Cu") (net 27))
 (segment (start 147.182 61.447) (end 147.182 78.0618) (width 0.5) (layer "B.Cu") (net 35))
 (segment (start 147.182 78.0618) (end 155.31 86.19) (width 0.5) (layer "B.Cu") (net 35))
 (segment (start 146.605 60.87) (end 147.182 61.447) (width 0.5) (layer "B.Cu") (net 35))
 (segment (start 160.5 79.5) (end 156.765 75.765) (width 0.5) (layer "B.Cu") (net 38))
 (segment (start 160.775454 81.775454) (end 160.5 81.5) (width 0.5) (layer "B.Cu") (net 38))
 (segment (start 165 85.47894) (end 164.999998 85.47894) (width 0.5) (layer "B.Cu") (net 38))
 (segment (start 160.5 81.5) (end 160.5 79.5) (width 0.5) (layer "B.Cu") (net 38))
 (segment (start 164 85) (end 160.775454 81.775454) (width 0.5) (layer "B.Cu") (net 38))
 (segment (start 156.765 75.765) (end 156.765 60.87) (width 0.5) (layer "B.Cu") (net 38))
 (segment (start 164.999998 85.47894) (end 164.521058 85) (width 0.5) (layer "B.Cu") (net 38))
 (segment (start 165 85.46) (end 165 85.47894) (width 0.5) (layer "B.Cu") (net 38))
 (segment (start 164.521058 85) (end 164 85) (width 0.5) (layer "B.Cu") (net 38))
 (segment (start 136.76 78.7077) (end 134.772 76.7195) (width 0.5) (layer "F.Cu") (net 1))
 (segment (start 127.052 69) (end 126.54 69) (width 0.5) (layer "F.Cu") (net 1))
 (segment (start 136.79102 78.73872) (end 136.76 78.7077) (width 0.5) (layer "F.Cu") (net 1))
 (segment (start 120.718 78.5607) (end 125.4393 78.5607) (width 0.5) (layer "F.Cu") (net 1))
 (segment (start 125.4393 78.5607) (end 131.026 72.974) (width 0.5) (layer "F.Cu") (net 1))
 (segment (start 114 85.2791) (end 120.718 78.5607) (width 0.5) (layer "F.Cu") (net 1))
 (segment (start 152.93892 78.73892) (end 152.93892 78.73872) (width 0.5) (layer "F.Cu") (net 1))
 (segment (start 114 86) (end 114 85.2791) (width 0.5) (layer "F.Cu") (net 1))
 (segment (start 130.335 72.283) (end 127.052 69) (width 0.5) (layer "F.Cu") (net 1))
 (segment (start 131.026 72.974) (end 130.335 72.283) (width 0.5) (layer "F.Cu") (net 1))
 (segment (start 155.31 81.11) (end 152.93892 78.73892) (width 0.5) (layer "F.Cu") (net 1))
 (segment (start 152.93892 78.73872) (end 136.79102 78.73872) (width 0.5) (layer "F.Cu") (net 1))
 (segment (start 134.772 76.7195) (end 130.335 72.283) (width 0.5) (layer "F.Cu") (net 1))
 (segment (start 131.0491 101.1941) (end 121.5096 101.1941) (width 0.5) (layer "B.Cu") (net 1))
 (segment (start 112 88) (end 114 86) (width 0.5) (layer "B.Cu") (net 1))
 (segment (start 121.5096 101.1941) (end 112 91.6845) (width 0.5) (layer "B.Cu") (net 1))
 (segment (start 138.985 109.13) (end 131.0491 101.1941) (width 0.5) (layer "B.Cu") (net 1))
 (segment (start 112 91.6845) (end 112 88) (width 0.5) (layer "B.Cu") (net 1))
 (segment (start 132.13 60.87) (end 132.385 60.87) (width 0.5) (layer "B.Cu") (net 24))
 (segment (start 124 69) (end 132.13 60.87) (width 0.5) (layer "B.Cu") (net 24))
 (segment (start 150.293 109.13) (end 148.163 107) (width 0.5) (layer "F.Cu") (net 3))
 (segment (start 151.685 109.13) (end 150.293 109.13) (width 0.5) (layer "F.Cu") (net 3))
 (segment (start 124 107) (end 114 97) (width 0.5) (layer "F.Cu") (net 3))
 (segment (start 148.163 107) (end 124 107) (width 0.5) (layer "F.Cu") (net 3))
 (segment (start 114 97) (end 114 91.08) (width 0.5) (layer "F.Cu") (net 3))
 (segment (start 163 62.025) (end 161.845 60.87) (width 0.5) (layer "B.Cu") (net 37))
 (segment (start 164.42 82.92) (end 163 81.5) (width 0.5) (layer "B.Cu") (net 37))
 (segment (start 163 81.5) (end 163 62.025) (width 0.5) (layer "B.Cu") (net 37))
 (segment (start 165 82.92) (end 164.42 82.92) (width 0.5) (layer "B.Cu") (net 37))
 (segment (start 159.305 98.775) (end 165 93.08) (width 0.5) (layer "B.Cu") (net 41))
 (segment (start 159.305 109.13) (end 159.305 98.775) (width 0.5) (layer "B.Cu") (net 41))
 (segment (start 152.202 61.387) (end 151.685 60.87) (width 0.5) (layer "B.Cu") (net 33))
 (segment (start 152.202 73.702) (end 152.202 61.387) (width 0.5) (layer "B.Cu") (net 33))
 (segment (start 153.384 74.884) (end 152.202 73.702) (width 0.5) (layer "B.Cu") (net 33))
 (segment (start 158.5 90.62) (end 158.5 80.189354) (width 0.5) (layer "B.Cu") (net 33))
 (segment (start 155.31 93.81) (end 158.5 90.62) (width 0.5) (layer "B.Cu") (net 33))
 (segment (start 158.5 80.189354) (end 153.384 75.073354) (width 0.5) (layer "B.Cu") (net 33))
 (segment (start 153.384 75.073354) (end 153.384 74.884) (width 0.5) (layer "B.Cu") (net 33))
 (segment (start 165 61.485) (end 164.385 60.87) (width 0.5) (layer "B.Cu") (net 36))
 (segment (start 165 80.38) (end 165 61.485) (width 0.5) (layer "B.Cu") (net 36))
 (segment (start 137.465 60.87) (end 137.465 63.2834) (width 0.5) (layer "B.Cu") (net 4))
 (segment (start 137.465 63.2834) (end 131.69 69.0584) (width 0.5) (layer "B.Cu") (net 4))
 (segment (start 131.69 69.0584) (end 131.69 69.5) (width 0.5) (layer "B.Cu") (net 4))
 (segment (start 139.31 69.5) (end 146.89 77.08) (width 0.5) (layer "F.Cu") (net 5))
 (segment (start 146.89 77.08) (end 160.5 77.08) (width 0.5) (layer "F.Cu") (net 5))
 (segment (start 146.54 74.54) (end 145.5 73.5) (width 0.5) (layer "F.Cu") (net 23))
 (segment (start 160.5 74.54) (end 146.54 74.54) (width 0.5) (layer "F.Cu") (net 23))
 (segment (start 150.85 69.46) (end 150.81 69.5) (width 0.5) (layer "F.Cu") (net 26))
 (segment (start 160.5 69.46) (end 150.85 69.46) (width 0.5) (layer "F.Cu") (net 26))
 (segment (start 144.12 96.2) (end 147.54 96.2) (width 0.5) (layer "F.Cu") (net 15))
 (segment (start 147.54 96.2) (end 147.69 96.35) (width 0.5) (layer "F.Cu") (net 15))
 (segment (start 147.69 86.19) (end 144.27 86.19) (width 0.5) (layer "F.Cu") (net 19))
 (segment (start 144.27 86.19) (end 144.12 86.04) (width 0.5) (layer "F.Cu") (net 19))
 (segment (start 144.27 83.65) (end 144.12 83.5) (width 0.5) (layer "F.Cu") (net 20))
 (segment (start 147.69 83.65) (end 144.27 83.65) (width 0.5) (layer "F.Cu") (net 20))
 (segment (start 147.69 93.81) (end 144.27 93.81) (width 0.5) (layer "F.Cu") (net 16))
 (segment (start 144.27 93.81) (end 144.12 93.66) (width 0.5) (layer "F.Cu") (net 16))
 (segment (start 144.12 91.12) (end 147.54 91.12) (width 0.5) (layer "F.Cu") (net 17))
 (segment (start 147.54 91.12) (end 147.69 91.27) (width 0.5) (layer "F.Cu") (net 17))
 (segment (start 147.54 88.58) (end 147.69 88.73) (width 0.5) (layer "F.Cu") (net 18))
 (segment (start 144.12 88.58) (end 147.54 88.58) (width 0.5) (layer "F.Cu") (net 18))
 (segment (start 147.54 80.96) (end 147.69 81.11) (width 0.5) (layer "B.Cu") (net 21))
 (segment (start 144.12 80.96) (end 147.54 80.96) (width 0.5) (layer "B.Cu") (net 21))
 (segment (start 149.93 89.03) (end 149.93 98.6181) (width 0.5) (layer "F.Cu") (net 14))
 (segment (start 148.266 100.282) (end 145.662 100.282) (width 0.5) (layer "F.Cu") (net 14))
 (segment (start 155.31 83.65) (end 149.93 89.03) (width 0.5) (layer "F.Cu") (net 14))
 (segment (start 149.93 98.6181) (end 148.266 100.282) (width 0.5) (layer "F.Cu") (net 14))
 (segment (start 145.662 100.282) (end 144.12 98.74) (width 0.5) (layer "F.Cu") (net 14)))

